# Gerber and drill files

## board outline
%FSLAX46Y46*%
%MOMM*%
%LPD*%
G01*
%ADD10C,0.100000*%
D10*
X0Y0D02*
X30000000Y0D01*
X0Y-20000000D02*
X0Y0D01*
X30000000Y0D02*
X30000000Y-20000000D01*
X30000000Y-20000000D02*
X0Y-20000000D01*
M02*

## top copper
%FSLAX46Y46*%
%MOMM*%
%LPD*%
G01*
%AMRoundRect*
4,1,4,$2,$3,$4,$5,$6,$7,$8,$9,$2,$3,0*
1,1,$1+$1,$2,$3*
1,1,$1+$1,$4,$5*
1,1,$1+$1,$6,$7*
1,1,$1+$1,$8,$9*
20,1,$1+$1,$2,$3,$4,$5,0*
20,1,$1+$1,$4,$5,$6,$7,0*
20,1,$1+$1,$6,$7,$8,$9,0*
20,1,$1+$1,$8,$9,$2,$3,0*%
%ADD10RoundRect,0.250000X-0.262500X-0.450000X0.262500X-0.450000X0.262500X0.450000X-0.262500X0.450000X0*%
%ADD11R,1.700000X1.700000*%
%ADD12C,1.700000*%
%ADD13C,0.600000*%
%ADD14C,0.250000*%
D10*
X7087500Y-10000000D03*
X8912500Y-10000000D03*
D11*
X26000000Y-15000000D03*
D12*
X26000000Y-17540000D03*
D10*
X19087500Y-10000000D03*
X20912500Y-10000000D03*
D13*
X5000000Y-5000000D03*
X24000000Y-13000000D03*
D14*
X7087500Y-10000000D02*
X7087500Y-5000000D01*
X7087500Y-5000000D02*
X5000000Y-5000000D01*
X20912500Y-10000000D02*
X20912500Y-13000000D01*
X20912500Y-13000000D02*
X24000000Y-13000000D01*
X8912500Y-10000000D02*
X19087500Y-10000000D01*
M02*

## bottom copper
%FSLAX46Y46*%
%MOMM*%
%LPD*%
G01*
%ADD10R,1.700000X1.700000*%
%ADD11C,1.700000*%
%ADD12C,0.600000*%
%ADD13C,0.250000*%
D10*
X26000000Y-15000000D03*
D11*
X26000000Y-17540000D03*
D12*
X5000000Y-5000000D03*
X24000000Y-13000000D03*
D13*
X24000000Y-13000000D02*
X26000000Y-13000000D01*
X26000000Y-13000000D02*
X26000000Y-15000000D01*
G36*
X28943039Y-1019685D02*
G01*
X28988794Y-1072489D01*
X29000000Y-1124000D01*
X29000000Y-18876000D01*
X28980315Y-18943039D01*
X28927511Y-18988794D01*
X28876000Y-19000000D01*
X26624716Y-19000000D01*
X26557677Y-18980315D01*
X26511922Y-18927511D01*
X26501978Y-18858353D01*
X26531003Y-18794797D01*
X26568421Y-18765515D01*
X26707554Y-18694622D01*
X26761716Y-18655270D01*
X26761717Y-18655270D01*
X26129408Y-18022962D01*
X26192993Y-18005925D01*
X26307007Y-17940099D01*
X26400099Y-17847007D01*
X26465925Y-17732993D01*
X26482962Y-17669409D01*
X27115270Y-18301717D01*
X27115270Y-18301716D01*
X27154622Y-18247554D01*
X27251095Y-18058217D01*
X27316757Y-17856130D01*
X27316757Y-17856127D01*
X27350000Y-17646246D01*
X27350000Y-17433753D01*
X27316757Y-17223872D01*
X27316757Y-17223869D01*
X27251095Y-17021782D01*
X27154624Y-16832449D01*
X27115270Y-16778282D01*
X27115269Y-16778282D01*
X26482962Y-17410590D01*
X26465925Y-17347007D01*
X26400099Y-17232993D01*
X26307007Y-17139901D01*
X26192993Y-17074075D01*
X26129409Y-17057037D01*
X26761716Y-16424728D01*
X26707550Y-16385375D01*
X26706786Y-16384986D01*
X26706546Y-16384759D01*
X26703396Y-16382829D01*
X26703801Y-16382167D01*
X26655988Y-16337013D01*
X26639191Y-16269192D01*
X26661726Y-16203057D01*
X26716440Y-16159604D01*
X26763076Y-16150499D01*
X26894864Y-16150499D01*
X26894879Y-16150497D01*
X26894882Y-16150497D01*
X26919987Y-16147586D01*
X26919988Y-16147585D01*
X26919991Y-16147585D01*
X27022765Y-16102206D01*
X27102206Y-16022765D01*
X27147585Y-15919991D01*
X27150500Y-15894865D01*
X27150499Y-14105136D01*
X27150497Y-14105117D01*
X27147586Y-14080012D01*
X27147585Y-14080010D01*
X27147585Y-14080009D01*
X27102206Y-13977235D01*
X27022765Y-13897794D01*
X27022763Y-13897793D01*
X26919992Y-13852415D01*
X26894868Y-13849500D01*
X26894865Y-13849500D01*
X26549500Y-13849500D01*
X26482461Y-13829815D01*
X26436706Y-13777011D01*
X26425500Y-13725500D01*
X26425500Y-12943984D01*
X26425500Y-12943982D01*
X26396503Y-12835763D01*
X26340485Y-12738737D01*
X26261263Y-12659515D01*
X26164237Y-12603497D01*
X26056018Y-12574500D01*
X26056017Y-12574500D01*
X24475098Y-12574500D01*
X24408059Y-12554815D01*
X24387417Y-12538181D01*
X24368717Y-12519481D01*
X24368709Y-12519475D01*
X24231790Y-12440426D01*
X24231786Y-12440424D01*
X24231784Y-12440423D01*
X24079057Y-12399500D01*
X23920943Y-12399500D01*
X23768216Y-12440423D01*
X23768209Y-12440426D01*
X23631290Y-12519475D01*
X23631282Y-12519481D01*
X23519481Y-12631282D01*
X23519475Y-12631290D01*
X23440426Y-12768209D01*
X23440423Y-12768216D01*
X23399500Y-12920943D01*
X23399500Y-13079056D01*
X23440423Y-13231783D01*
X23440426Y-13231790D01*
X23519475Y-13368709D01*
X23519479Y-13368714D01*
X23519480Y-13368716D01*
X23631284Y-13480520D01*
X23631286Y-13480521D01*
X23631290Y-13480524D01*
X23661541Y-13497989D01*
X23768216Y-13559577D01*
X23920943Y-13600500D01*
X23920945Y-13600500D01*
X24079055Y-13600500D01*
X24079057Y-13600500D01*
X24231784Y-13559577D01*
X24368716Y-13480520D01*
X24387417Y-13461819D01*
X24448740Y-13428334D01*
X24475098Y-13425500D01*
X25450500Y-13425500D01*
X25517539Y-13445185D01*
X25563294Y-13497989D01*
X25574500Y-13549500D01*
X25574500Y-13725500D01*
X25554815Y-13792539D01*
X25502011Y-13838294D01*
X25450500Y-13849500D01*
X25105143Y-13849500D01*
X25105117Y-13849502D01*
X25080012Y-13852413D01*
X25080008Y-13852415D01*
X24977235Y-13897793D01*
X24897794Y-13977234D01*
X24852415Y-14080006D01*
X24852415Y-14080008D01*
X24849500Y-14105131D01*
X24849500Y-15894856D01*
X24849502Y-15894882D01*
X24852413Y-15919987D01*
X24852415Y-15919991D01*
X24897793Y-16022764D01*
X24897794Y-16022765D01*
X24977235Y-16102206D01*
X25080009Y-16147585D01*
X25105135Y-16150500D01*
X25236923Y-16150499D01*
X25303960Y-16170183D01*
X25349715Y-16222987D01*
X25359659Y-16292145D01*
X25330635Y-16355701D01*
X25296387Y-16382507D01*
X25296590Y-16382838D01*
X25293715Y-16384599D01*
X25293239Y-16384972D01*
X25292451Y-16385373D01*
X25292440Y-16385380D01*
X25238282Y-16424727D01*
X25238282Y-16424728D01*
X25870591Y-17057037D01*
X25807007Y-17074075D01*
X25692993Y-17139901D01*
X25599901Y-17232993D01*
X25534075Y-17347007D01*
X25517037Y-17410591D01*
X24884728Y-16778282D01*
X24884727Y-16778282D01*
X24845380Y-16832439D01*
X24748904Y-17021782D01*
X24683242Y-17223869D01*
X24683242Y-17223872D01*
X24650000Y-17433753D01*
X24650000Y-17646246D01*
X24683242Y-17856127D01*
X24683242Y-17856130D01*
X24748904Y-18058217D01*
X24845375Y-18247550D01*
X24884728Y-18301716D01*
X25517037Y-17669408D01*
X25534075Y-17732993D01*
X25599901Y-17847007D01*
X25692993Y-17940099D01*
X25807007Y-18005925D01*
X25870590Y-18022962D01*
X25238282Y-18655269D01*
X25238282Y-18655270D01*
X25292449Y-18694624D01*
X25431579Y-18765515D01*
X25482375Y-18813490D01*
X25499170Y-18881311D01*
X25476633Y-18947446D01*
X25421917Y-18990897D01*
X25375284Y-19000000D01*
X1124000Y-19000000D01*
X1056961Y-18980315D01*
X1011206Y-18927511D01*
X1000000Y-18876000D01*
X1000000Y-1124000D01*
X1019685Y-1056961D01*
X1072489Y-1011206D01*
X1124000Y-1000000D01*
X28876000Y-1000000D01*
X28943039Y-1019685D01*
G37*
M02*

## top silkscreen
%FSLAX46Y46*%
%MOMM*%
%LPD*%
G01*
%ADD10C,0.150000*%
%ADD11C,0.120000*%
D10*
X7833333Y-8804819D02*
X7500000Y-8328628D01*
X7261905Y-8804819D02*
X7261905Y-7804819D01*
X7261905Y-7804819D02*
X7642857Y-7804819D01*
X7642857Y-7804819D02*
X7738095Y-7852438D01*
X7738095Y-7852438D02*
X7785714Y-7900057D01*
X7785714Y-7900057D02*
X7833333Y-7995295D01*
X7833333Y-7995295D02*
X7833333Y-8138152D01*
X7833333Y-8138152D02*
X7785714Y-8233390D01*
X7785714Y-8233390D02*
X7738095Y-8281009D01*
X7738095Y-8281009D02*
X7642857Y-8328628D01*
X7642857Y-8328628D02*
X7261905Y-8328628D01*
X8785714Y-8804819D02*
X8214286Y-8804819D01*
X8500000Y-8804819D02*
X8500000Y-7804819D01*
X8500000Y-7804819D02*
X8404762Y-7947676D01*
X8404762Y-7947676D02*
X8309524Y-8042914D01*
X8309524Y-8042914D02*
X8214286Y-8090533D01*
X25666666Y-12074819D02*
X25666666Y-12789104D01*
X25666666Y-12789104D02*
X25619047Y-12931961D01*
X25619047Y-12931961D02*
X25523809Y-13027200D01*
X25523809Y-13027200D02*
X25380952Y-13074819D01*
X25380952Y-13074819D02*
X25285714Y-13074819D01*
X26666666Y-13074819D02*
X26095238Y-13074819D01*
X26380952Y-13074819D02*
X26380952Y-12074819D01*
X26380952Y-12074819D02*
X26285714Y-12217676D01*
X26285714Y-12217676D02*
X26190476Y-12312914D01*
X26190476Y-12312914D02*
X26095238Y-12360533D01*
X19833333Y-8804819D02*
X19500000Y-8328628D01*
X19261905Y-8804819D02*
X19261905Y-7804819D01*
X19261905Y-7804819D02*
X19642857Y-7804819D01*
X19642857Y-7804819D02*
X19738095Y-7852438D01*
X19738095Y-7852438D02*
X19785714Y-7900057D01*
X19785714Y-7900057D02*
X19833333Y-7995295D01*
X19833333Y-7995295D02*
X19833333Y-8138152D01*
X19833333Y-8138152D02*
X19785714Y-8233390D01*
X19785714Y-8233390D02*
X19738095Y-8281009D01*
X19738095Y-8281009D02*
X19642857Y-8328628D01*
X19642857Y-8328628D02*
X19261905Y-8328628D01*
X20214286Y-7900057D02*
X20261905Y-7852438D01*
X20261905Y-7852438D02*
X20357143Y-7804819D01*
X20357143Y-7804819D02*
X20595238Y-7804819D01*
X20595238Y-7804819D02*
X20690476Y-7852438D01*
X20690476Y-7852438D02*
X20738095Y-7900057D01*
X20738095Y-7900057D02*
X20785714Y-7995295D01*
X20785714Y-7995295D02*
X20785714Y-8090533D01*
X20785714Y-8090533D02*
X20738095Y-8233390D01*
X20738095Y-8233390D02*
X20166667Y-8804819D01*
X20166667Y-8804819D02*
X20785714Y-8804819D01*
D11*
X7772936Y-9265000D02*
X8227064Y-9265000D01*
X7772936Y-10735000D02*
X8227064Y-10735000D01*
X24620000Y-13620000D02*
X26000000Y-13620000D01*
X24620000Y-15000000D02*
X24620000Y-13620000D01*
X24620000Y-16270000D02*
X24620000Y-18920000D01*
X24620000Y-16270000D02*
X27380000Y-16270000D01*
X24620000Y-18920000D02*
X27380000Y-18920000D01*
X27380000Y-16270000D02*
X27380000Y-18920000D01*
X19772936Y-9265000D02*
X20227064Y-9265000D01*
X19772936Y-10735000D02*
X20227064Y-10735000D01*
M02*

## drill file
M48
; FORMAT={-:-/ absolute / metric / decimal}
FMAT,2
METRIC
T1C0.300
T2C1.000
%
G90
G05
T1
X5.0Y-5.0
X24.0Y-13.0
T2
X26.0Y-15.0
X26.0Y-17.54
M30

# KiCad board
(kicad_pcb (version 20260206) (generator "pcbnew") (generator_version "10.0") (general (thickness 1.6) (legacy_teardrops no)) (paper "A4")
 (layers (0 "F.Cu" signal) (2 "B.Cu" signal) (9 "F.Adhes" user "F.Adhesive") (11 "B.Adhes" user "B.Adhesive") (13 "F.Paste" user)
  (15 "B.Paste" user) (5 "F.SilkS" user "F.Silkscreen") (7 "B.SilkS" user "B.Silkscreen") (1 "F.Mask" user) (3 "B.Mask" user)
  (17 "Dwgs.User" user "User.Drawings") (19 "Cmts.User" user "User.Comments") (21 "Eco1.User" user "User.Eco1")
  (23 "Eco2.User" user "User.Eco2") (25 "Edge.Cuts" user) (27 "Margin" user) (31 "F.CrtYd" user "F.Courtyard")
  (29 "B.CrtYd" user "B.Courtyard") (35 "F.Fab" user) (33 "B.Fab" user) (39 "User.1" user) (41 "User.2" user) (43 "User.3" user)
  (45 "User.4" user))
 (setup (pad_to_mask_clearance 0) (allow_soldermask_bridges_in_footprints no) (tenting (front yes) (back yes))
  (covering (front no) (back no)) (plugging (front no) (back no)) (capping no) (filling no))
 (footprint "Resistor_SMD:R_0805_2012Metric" (layer "F.Cu") (at 8 10)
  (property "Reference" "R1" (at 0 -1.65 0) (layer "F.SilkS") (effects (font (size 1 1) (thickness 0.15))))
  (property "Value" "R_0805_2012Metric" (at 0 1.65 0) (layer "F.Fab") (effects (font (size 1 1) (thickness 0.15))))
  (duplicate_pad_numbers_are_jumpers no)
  (fp_line (start -0.227064 -0.735) (end 0.227064 -0.735) (stroke (width 0.12) (type solid)) (layer "F.SilkS"))
  (fp_line (start -0.227064 0.735) (end 0.227064 0.735) (stroke (width 0.12) (type solid)) (layer "F.SilkS"))
  (pad "1" smd roundrect (at -0.9125 0) (size 1.025 1.4) (layers "F.Cu" "F.Mask" "F.Paste") (roundrect_rratio 0.243902) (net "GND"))
  (pad "2" smd roundrect (at 0.9125 0) (size 1.025 1.4) (layers "F.Cu" "F.Mask" "F.Paste") (roundrect_rratio 0.243902) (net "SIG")))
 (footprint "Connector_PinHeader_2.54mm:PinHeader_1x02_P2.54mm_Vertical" (layer "F.Cu") (at 26 15)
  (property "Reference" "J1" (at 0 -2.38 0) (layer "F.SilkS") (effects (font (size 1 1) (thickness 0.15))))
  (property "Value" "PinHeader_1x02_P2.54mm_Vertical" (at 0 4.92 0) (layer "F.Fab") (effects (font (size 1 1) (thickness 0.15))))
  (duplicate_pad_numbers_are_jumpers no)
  (fp_line (start -1.38 -1.38) (end 0 -1.38) (stroke (width 0.12) (type solid)) (layer "F.SilkS"))
  (fp_line (start -1.38 0) (end -1.38 -1.38) (stroke (width 0.12) (type solid)) (layer "F.SilkS"))
  (fp_line (start -1.38 1.27) (end -1.38 3.92) (stroke (width 0.12) (type solid)) (layer "F.SilkS"))
  (fp_line (start -1.38 1.27) (end 1.38 1.27) (stroke (width 0.12) (type solid)) (layer "F.SilkS"))
  (fp_line (start -1.38 3.92) (end 1.38 3.92) (stroke (width 0.12) (type solid)) (layer "F.SilkS"))
  (fp_line (start 1.38 1.27) (end 1.38 3.92) (stroke (width 0.12) (type solid)) (layer "F.SilkS"))
  (pad "1" thru_hole rect (at 0 0) (size 1.7 1.7) (drill 1) (layers "*.Cu" "*.Mask") (remove_unused_layers no) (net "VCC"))
  (pad "2" thru_hole circle (at 0 2.54) (size 1.7 1.7) (drill 1) (layers "*.Cu" "*.Mask") (remove_unused_layers no) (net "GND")))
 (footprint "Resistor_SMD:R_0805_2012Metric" (layer "F.Cu") (at 20 10)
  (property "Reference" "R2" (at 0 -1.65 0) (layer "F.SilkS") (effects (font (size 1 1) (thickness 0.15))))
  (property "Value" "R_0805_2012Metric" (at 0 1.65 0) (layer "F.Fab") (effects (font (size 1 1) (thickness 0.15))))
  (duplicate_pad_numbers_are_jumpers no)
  (fp_line (start -0.227064 -0.735) (end 0.227064 -0.735) (stroke (width 0.12) (type solid)) (layer "F.SilkS"))
  (fp_line (start -0.227064 0.735) (end 0.227064 0.735) (stroke (width 0.12) (type solid)) (layer "F.SilkS"))
  (pad "1" smd roundrect (at -0.9125 0) (size 1.025 1.4) (layers "F.Cu" "F.Mask" "F.Paste") (roundrect_rratio 0.243902) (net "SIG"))
  (pad "2" smd roundrect (at 0.9125 0) (size 1.025 1.4) (layers "F.Cu" "F.Mask" "F.Paste") (roundrect_rratio 0.243902) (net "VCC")))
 (gr_line (start 0 0) (end 30 0) (stroke (width 0.1) (type default)) (layer "Edge.Cuts"))
 (gr_line (start 0 20) (end 0 0) (stroke (width 0.1) (type default)) (layer "Edge.Cuts"))
 (gr_line (start 30 0) (end 30 20) (stroke (width 0.1) (type default)) (layer "Edge.Cuts"))
 (gr_line (start 30 20) (end 0 20) (stroke (width 0.1) (type default)) (layer "Edge.Cuts"))
 (segment (start 7.0875 10) (end 7.0875 5) (width 0.25) (layer "F.Cu") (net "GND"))
 (segment (start 7.0875 5) (end 5 5) (width 0.25) (layer "F.Cu") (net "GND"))
 (via (at 5 5) (size 0.6) (drill 0.3) (layers "F.Cu" "B.Cu") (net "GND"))
 (segment (start 20.9125 10) (end 20.9125 13) (width 0.25) (layer "F.Cu") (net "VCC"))
 (segment (start 20.9125 13) (end 24 13) (width 0.25) (layer "F.Cu") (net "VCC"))
 (via (at 24 13) (size 0.6) (drill 0.3) (layers "F.Cu" "B.Cu") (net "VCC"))
 (segment (start 24 13) (end 26 13) (width 0.25) (layer "B.Cu") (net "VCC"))
 (segment (start 26 13) (end 26 15) (width 0.25) (layer "B.Cu") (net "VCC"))
 (segment (start 8.9125 10) (end 19.0875 10) (width 0.25) (layer "F.Cu") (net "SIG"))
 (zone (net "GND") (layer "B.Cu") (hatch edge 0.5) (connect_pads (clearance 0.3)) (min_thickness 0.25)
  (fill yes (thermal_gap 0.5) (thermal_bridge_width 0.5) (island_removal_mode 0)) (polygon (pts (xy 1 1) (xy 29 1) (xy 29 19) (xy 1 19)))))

